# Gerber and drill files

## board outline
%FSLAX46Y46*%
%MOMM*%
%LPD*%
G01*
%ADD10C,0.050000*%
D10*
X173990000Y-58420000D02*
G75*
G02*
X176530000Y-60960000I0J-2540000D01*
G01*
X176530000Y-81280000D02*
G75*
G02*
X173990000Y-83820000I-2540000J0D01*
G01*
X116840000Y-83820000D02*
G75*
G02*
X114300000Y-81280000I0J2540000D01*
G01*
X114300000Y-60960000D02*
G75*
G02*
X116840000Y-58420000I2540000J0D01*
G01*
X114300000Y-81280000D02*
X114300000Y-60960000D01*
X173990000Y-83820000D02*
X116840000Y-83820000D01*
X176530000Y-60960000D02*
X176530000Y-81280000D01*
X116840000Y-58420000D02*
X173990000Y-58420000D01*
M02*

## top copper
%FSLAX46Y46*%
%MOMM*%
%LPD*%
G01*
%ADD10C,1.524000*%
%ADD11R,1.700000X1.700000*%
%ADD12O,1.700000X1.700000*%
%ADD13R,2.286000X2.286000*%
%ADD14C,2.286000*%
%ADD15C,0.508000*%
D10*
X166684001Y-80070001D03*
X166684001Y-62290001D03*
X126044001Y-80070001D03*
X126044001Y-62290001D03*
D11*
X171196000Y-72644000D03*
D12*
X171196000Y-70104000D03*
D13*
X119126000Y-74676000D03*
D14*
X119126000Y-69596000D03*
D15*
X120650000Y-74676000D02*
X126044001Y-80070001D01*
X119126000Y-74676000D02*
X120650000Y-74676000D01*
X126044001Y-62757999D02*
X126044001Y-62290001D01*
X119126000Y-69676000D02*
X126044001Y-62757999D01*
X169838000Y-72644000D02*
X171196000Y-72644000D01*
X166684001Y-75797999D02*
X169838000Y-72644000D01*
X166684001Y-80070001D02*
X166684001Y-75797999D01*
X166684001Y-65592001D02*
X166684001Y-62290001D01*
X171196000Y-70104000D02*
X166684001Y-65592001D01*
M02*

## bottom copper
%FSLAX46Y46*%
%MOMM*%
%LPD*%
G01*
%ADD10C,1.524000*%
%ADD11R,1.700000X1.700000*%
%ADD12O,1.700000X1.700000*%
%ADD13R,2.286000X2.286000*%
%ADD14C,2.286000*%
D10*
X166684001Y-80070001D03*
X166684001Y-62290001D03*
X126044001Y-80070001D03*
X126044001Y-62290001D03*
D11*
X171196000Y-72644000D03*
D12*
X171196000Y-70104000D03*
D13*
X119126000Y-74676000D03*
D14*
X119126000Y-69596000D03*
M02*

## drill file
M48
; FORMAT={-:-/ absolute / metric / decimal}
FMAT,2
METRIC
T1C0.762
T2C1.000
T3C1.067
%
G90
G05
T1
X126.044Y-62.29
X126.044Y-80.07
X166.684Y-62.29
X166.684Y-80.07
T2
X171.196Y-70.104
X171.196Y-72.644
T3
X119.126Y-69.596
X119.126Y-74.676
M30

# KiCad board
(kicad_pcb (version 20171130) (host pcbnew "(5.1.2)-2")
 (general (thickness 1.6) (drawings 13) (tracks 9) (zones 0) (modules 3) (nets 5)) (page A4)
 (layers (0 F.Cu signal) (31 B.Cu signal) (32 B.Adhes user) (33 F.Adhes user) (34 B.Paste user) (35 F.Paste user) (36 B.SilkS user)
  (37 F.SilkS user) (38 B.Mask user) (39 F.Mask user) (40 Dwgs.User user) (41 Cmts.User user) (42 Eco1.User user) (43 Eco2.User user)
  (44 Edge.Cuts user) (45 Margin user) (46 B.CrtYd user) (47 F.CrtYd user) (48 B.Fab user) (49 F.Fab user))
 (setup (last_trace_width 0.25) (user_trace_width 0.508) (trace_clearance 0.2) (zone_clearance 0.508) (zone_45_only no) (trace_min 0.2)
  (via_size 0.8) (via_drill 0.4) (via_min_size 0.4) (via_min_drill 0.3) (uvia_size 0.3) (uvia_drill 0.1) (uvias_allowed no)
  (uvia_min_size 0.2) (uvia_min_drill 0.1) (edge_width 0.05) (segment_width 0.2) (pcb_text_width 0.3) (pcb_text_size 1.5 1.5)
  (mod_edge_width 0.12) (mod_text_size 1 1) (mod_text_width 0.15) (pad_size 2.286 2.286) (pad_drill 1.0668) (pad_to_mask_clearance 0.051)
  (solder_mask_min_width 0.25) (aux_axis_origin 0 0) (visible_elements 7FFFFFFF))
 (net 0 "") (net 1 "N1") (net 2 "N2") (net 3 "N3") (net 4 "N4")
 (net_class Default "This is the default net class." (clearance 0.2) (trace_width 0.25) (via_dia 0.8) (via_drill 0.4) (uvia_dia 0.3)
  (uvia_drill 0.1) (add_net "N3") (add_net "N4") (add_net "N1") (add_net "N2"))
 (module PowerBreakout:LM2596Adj (layer F.Cu) (at 148.904001 72.450001)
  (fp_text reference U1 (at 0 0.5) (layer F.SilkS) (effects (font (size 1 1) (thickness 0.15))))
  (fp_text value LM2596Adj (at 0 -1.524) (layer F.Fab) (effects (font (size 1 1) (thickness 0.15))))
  (pad 4 thru_hole circle (at 17.78 7.62) (size 1.524 1.524) (drill 0.762) (layers *.Cu *.Mask) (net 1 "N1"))
  (pad 3 thru_hole circle (at 17.78 -10.16) (size 1.524 1.524) (drill 0.762) (layers *.Cu *.Mask) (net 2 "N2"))
  (pad 2 thru_hole circle (at -22.86 7.62) (size 1.524 1.524) (drill 0.762) (layers *.Cu *.Mask) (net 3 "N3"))
  (pad 1 thru_hole circle (at -22.86 -10.16) (size 1.524 1.524) (drill 0.762) (layers *.Cu *.Mask) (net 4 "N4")))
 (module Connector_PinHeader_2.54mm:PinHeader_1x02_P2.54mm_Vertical (layer F.Cu) (at 171.196 72.644 180)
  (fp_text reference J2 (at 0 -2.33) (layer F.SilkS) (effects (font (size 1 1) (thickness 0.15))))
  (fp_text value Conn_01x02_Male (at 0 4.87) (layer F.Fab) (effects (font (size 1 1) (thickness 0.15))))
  (pad 1 thru_hole rect (at 0 0 180) (size 1.7 1.7) (drill 1) (layers *.Cu *.Mask) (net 1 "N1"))
  (pad 2 thru_hole oval (at 0 2.54 180) (size 1.7 1.7) (drill 1) (layers *.Cu *.Mask) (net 2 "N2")))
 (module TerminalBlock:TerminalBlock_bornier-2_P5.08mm (layer F.Cu) (at 119.126 74.676 90)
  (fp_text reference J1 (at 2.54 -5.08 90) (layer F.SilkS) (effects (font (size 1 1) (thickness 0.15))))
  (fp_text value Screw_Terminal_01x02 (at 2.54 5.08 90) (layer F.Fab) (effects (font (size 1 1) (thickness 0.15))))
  (pad 1 thru_hole rect (at 0 0 90) (size 2.286 2.286) (drill 1.0668) (layers *.Cu *.Mask) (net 3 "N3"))
  (pad 2 thru_hole circle (at 5.08 0 90) (size 2.286 2.286) (drill 1.0668) (layers *.Cu *.Mask) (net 4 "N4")))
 (gr_arc (start 173.99 60.96) (end 176.53 60.96) (angle -90) (layer Edge.Cuts) (width 0.05))
 (gr_arc (start 173.99 81.28) (end 173.99 83.82) (angle -90) (layer Edge.Cuts) (width 0.05))
 (gr_arc (start 116.84 81.28) (end 114.3 81.28) (angle -90) (layer Edge.Cuts) (width 0.05))
 (gr_arc (start 116.84 60.96) (end 116.84 58.42) (angle -90) (layer Edge.Cuts) (width 0.05))
 (gr_line (start 114.3 81.28) (end 114.3 60.96) (layer Edge.Cuts) (width 0.05))
 (gr_line (start 173.99 83.82) (end 116.84 83.82) (layer Edge.Cuts) (width 0.05))
 (gr_line (start 176.53 60.96) (end 176.53 81.28) (layer Edge.Cuts) (width 0.05))
 (gr_line (start 116.84 58.42) (end 173.99 58.42) (layer Edge.Cuts) (width 0.05))
 (segment (start 120.65 74.676) (end 126.044001 80.070001) (width 0.508) (layer F.Cu) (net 3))
 (segment (start 119.126 74.676) (end 120.65 74.676) (width 0.508) (layer F.Cu) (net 3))
 (segment (start 126.044001 62.757999) (end 126.044001 62.290001) (width 0.508) (layer F.Cu) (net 4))
 (segment (start 119.126 69.676) (end 126.044001 62.757999) (width 0.508) (layer F.Cu) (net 4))
 (segment (start 169.838 72.644) (end 171.196 72.644) (width 0.508) (layer F.Cu) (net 1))
 (segment (start 166.684001 75.797999) (end 169.838 72.644) (width 0.508) (layer F.Cu) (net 1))
 (segment (start 166.684001 80.070001) (end 166.684001 75.797999) (width 0.508) (layer F.Cu) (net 1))
 (segment (start 166.684001 65.592001) (end 166.684001 62.290001) (width 0.508) (layer F.Cu) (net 2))
 (segment (start 171.196 70.104) (end 166.684001 65.592001) (width 0.508) (layer F.Cu) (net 2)))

